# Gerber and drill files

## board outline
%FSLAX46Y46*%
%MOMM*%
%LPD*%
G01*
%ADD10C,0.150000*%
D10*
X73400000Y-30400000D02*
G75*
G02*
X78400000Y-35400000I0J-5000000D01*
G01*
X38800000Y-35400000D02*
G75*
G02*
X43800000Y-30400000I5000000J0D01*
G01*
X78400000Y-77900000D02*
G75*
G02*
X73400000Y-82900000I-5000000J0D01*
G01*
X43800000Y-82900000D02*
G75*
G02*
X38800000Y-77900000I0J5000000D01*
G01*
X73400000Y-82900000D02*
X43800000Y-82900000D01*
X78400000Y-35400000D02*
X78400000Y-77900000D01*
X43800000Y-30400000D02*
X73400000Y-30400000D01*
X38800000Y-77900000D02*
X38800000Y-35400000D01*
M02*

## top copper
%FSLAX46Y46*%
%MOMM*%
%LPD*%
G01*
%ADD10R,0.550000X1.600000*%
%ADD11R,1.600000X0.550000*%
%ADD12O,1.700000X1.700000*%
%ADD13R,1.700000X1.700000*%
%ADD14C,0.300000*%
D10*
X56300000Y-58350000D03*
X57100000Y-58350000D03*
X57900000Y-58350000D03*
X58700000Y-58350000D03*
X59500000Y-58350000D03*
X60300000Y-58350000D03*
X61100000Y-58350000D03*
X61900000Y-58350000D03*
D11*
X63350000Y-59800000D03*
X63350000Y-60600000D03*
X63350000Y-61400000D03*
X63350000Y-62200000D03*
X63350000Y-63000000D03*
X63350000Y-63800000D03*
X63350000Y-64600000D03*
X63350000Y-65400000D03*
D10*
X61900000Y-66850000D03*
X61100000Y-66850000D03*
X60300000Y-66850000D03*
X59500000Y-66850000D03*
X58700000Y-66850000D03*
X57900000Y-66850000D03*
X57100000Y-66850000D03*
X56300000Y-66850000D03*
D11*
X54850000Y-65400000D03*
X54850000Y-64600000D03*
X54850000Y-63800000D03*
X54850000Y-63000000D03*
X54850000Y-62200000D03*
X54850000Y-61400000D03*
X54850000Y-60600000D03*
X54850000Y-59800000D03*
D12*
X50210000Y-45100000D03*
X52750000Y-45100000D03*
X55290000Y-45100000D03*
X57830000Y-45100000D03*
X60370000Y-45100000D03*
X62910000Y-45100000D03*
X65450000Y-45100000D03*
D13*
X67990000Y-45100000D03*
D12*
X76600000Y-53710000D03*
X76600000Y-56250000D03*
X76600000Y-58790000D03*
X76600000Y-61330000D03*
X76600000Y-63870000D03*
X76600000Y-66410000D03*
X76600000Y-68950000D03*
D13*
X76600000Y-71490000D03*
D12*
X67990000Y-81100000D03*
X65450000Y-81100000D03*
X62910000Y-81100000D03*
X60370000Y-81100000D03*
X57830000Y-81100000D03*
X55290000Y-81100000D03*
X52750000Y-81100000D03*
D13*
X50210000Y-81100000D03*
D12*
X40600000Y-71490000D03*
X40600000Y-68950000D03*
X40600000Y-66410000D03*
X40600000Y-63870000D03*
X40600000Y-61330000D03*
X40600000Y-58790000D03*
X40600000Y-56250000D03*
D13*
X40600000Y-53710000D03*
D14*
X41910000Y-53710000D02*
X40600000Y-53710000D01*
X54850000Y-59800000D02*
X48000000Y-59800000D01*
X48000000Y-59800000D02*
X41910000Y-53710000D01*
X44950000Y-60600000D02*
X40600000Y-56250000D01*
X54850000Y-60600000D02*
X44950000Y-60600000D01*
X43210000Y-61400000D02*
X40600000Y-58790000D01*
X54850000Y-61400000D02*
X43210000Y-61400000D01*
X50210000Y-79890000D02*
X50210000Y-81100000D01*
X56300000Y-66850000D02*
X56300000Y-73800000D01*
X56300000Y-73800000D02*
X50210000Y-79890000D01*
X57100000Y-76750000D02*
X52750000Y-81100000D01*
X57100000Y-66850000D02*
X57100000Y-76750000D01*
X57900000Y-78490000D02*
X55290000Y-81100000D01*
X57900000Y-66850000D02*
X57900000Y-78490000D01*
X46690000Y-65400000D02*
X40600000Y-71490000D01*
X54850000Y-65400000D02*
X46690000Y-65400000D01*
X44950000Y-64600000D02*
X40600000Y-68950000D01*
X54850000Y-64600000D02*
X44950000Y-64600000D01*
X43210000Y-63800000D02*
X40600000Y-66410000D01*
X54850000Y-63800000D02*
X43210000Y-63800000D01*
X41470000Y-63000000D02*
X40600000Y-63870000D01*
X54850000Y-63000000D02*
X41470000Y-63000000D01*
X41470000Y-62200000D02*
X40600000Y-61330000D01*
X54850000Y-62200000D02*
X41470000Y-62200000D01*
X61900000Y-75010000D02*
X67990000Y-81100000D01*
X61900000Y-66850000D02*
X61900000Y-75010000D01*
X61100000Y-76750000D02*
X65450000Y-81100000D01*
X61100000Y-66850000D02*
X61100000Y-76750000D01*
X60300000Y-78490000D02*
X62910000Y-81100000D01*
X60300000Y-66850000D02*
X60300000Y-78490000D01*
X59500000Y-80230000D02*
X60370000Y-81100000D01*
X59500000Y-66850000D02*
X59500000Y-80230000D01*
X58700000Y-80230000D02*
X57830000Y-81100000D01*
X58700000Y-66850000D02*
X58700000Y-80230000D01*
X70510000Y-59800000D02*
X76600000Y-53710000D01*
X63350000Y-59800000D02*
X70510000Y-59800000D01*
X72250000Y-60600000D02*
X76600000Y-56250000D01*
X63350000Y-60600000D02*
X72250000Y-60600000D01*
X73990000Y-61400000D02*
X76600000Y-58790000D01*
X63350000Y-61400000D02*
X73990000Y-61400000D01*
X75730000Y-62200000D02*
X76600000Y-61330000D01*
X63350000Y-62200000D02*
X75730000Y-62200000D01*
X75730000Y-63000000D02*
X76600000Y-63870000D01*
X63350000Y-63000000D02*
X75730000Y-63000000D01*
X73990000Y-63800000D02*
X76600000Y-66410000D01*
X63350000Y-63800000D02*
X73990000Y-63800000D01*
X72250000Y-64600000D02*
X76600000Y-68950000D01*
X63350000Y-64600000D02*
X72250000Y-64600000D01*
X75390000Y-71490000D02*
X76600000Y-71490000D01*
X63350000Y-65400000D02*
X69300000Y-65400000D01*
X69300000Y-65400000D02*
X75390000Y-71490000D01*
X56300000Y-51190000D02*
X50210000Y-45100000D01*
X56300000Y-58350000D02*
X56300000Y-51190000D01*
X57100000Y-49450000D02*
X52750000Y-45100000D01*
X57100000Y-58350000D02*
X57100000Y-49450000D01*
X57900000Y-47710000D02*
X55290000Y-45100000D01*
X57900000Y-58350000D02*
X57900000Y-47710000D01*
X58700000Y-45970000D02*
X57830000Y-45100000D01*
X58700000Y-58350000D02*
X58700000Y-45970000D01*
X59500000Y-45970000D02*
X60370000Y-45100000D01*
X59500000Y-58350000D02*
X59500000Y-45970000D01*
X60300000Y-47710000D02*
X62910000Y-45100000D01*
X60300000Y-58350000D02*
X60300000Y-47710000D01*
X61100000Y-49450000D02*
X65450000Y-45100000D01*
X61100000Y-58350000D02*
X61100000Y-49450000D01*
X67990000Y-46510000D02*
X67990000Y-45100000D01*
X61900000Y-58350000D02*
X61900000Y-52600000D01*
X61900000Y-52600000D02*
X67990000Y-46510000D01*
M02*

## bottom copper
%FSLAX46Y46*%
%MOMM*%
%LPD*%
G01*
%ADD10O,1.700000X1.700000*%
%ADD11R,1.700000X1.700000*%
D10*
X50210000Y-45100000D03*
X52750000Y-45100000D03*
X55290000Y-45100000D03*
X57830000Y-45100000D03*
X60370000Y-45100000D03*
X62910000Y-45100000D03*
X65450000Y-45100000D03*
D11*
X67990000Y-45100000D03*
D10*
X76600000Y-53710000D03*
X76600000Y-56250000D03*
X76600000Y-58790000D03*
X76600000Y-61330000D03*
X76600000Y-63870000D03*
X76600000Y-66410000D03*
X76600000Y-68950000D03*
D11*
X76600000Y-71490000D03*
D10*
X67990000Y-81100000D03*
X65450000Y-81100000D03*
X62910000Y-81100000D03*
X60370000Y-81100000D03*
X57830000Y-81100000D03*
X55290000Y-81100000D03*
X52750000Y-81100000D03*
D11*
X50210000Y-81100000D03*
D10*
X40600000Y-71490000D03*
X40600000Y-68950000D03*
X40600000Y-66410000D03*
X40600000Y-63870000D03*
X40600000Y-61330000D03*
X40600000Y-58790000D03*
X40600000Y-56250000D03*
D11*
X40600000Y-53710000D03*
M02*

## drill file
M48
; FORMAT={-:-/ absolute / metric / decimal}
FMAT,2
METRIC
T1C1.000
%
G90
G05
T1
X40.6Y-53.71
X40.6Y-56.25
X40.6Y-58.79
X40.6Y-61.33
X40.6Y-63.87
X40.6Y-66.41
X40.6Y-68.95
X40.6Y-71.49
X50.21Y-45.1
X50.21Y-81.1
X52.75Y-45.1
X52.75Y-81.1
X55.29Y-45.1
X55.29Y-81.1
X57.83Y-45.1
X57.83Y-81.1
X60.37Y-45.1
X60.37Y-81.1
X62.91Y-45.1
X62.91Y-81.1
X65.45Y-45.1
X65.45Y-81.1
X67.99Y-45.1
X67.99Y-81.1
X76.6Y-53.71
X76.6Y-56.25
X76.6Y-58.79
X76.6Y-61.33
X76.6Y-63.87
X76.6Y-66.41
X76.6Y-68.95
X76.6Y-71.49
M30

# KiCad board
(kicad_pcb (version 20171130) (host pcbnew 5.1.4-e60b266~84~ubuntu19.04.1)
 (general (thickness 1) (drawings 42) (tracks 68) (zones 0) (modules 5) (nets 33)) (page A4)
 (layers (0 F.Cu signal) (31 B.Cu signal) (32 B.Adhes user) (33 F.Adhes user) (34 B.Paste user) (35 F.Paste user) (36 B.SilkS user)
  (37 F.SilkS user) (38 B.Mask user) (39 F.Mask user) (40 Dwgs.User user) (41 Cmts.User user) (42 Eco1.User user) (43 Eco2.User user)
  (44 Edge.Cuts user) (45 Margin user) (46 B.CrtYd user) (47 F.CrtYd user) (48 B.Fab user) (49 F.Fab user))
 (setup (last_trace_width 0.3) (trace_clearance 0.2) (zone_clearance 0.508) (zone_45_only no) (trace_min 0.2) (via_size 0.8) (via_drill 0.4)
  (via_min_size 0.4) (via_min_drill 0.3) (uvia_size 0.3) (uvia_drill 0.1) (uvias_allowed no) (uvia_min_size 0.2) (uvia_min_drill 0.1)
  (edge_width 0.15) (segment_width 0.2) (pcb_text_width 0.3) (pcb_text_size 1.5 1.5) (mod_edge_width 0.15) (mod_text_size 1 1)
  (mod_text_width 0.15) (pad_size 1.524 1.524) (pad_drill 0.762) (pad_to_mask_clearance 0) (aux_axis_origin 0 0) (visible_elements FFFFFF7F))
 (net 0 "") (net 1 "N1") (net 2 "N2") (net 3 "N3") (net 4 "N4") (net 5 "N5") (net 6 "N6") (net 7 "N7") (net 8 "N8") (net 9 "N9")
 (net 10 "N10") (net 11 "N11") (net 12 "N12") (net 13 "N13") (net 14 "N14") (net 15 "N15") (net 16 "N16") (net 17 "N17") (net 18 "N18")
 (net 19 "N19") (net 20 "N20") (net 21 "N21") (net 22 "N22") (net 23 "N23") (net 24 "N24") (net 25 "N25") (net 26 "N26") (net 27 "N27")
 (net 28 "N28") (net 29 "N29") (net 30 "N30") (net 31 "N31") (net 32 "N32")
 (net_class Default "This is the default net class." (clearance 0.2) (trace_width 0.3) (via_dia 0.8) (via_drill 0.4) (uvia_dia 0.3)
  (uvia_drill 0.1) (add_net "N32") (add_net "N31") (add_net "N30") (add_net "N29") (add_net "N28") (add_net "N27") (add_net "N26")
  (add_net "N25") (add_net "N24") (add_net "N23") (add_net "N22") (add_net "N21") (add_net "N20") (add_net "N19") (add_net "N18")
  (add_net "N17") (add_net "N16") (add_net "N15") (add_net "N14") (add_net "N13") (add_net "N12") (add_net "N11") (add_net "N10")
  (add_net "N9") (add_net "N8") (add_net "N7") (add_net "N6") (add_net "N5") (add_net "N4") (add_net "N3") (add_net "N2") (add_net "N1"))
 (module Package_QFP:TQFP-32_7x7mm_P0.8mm (layer F.Cu) (at 59.1 62.6)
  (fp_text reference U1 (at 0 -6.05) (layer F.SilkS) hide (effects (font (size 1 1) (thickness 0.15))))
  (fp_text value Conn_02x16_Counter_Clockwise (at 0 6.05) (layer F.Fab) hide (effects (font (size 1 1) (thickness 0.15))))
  (pad 32 smd rect (at -2.8 -4.25 90) (size 1.6 0.55) (layers F.Cu F.Paste F.Mask) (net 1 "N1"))
  (pad 31 smd rect (at -2 -4.25 90) (size 1.6 0.55) (layers F.Cu F.Paste F.Mask) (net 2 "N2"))
  (pad 30 smd rect (at -1.2 -4.25 90) (size 1.6 0.55) (layers F.Cu F.Paste F.Mask) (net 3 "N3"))
  (pad 29 smd rect (at -0.4 -4.25 90) (size 1.6 0.55) (layers F.Cu F.Paste F.Mask) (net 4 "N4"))
  (pad 28 smd rect (at 0.4 -4.25 90) (size 1.6 0.55) (layers F.Cu F.Paste F.Mask) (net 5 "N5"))
  (pad 27 smd rect (at 1.2 -4.25 90) (size 1.6 0.55) (layers F.Cu F.Paste F.Mask) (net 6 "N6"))
  (pad 26 smd rect (at 2 -4.25 90) (size 1.6 0.55) (layers F.Cu F.Paste F.Mask) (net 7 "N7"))
  (pad 25 smd rect (at 2.8 -4.25 90) (size 1.6 0.55) (layers F.Cu F.Paste F.Mask) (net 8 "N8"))
  (pad 24 smd rect (at 4.25 -2.8) (size 1.6 0.55) (layers F.Cu F.Paste F.Mask) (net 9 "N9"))
  (pad 23 smd rect (at 4.25 -2) (size 1.6 0.55) (layers F.Cu F.Paste F.Mask) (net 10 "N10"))
  (pad 22 smd rect (at 4.25 -1.2) (size 1.6 0.55) (layers F.Cu F.Paste F.Mask) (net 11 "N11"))
  (pad 21 smd rect (at 4.25 -0.4) (size 1.6 0.55) (layers F.Cu F.Paste F.Mask) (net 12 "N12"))
  (pad 20 smd rect (at 4.25 0.4) (size 1.6 0.55) (layers F.Cu F.Paste F.Mask) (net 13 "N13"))
  (pad 19 smd rect (at 4.25 1.2) (size 1.6 0.55) (layers F.Cu F.Paste F.Mask) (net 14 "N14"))
  (pad 18 smd rect (at 4.25 2) (size 1.6 0.55) (layers F.Cu F.Paste F.Mask) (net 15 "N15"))
  (pad 17 smd rect (at 4.25 2.8) (size 1.6 0.55) (layers F.Cu F.Paste F.Mask) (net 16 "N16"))
  (pad 16 smd rect (at 2.8 4.25 90) (size 1.6 0.55) (layers F.Cu F.Paste F.Mask) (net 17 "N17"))
  (pad 15 smd rect (at 2 4.25 90) (size 1.6 0.55) (layers F.Cu F.Paste F.Mask) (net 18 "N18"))
  (pad 14 smd rect (at 1.2 4.25 90) (size 1.6 0.55) (layers F.Cu F.Paste F.Mask) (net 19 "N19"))
  (pad 13 smd rect (at 0.4 4.25 90) (size 1.6 0.55) (layers F.Cu F.Paste F.Mask) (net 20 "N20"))
  (pad 12 smd rect (at -0.4 4.25 90) (size 1.6 0.55) (layers F.Cu F.Paste F.Mask) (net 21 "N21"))
  (pad 11 smd rect (at -1.2 4.25 90) (size 1.6 0.55) (layers F.Cu F.Paste F.Mask) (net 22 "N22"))
  (pad 10 smd rect (at -2 4.25 90) (size 1.6 0.55) (layers F.Cu F.Paste F.Mask) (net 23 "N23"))
  (pad 9 smd rect (at -2.8 4.25 90) (size 1.6 0.55) (layers F.Cu F.Paste F.Mask) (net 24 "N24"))
  (pad 8 smd rect (at -4.25 2.8) (size 1.6 0.55) (layers F.Cu F.Paste F.Mask) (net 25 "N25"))
  (pad 7 smd rect (at -4.25 2) (size 1.6 0.55) (layers F.Cu F.Paste F.Mask) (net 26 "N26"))
  (pad 6 smd rect (at -4.25 1.2) (size 1.6 0.55) (layers F.Cu F.Paste F.Mask) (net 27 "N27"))
  (pad 5 smd rect (at -4.25 0.4) (size 1.6 0.55) (layers F.Cu F.Paste F.Mask) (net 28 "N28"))
  (pad 4 smd rect (at -4.25 -0.4) (size 1.6 0.55) (layers F.Cu F.Paste F.Mask) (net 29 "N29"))
  (pad 3 smd rect (at -4.25 -1.2) (size 1.6 0.55) (layers F.Cu F.Paste F.Mask) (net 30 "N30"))
  (pad 2 smd rect (at -4.25 -2) (size 1.6 0.55) (layers F.Cu F.Paste F.Mask) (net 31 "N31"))
  (pad 1 smd rect (at -4.25 -2.8) (size 1.6 0.55) (layers F.Cu F.Paste F.Mask) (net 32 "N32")))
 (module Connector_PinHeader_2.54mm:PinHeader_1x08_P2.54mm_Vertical (layer F.Cu) (at 67.99 45.1 270)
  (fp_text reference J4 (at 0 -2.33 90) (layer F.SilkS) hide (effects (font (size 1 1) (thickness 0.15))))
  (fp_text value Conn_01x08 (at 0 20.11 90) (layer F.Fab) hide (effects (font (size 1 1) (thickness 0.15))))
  (pad 8 thru_hole oval (at 0 17.78 270) (size 1.7 1.7) (drill 1) (layers *.Cu *.Mask) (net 1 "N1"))
  (pad 7 thru_hole oval (at 0 15.24 270) (size 1.7 1.7) (drill 1) (layers *.Cu *.Mask) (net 2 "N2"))
  (pad 6 thru_hole oval (at 0 12.7 270) (size 1.7 1.7) (drill 1) (layers *.Cu *.Mask) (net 3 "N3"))
  (pad 5 thru_hole oval (at 0 10.16 270) (size 1.7 1.7) (drill 1) (layers *.Cu *.Mask) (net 4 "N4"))
  (pad 4 thru_hole oval (at 0 7.62 270) (size 1.7 1.7) (drill 1) (layers *.Cu *.Mask) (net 5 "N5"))
  (pad 3 thru_hole oval (at 0 5.08 270) (size 1.7 1.7) (drill 1) (layers *.Cu *.Mask) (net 6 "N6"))
  (pad 2 thru_hole oval (at 0 2.54 270) (size 1.7 1.7) (drill 1) (layers *.Cu *.Mask) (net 7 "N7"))
  (pad 1 thru_hole rect (at 0 0 270) (size 1.7 1.7) (drill 1) (layers *.Cu *.Mask) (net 8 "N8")))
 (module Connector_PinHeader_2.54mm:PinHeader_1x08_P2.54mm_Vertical (layer F.Cu) (at 76.6 71.49 180)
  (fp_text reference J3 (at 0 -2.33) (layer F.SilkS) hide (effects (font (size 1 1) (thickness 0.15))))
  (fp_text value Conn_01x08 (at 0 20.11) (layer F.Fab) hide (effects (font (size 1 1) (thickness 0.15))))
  (pad 8 thru_hole oval (at 0 17.78 180) (size 1.7 1.7) (drill 1) (layers *.Cu *.Mask) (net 9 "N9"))
  (pad 7 thru_hole oval (at 0 15.24 180) (size 1.7 1.7) (drill 1) (layers *.Cu *.Mask) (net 10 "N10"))
  (pad 6 thru_hole oval (at 0 12.7 180) (size 1.7 1.7) (drill 1) (layers *.Cu *.Mask) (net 11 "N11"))
  (pad 5 thru_hole oval (at 0 10.16 180) (size 1.7 1.7) (drill 1) (layers *.Cu *.Mask) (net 12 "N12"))
  (pad 4 thru_hole oval (at 0 7.62 180) (size 1.7 1.7) (drill 1) (layers *.Cu *.Mask) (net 13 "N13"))
  (pad 3 thru_hole oval (at 0 5.08 180) (size 1.7 1.7) (drill 1) (layers *.Cu *.Mask) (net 14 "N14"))
  (pad 2 thru_hole oval (at 0 2.54 180) (size 1.7 1.7) (drill 1) (layers *.Cu *.Mask) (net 15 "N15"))
  (pad 1 thru_hole rect (at 0 0 180) (size 1.7 1.7) (drill 1) (layers *.Cu *.Mask) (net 16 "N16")))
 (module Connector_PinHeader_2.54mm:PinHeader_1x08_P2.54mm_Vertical (layer F.Cu) (at 50.21 81.1 90)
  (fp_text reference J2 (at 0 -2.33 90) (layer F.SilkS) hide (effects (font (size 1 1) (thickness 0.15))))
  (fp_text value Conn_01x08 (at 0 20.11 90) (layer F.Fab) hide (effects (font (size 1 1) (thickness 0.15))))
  (pad 8 thru_hole oval (at 0 17.78 90) (size 1.7 1.7) (drill 1) (layers *.Cu *.Mask) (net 17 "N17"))
  (pad 7 thru_hole oval (at 0 15.24 90) (size 1.7 1.7) (drill 1) (layers *.Cu *.Mask) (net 18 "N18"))
  (pad 6 thru_hole oval (at 0 12.7 90) (size 1.7 1.7) (drill 1) (layers *.Cu *.Mask) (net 19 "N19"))
  (pad 5 thru_hole oval (at 0 10.16 90) (size 1.7 1.7) (drill 1) (layers *.Cu *.Mask) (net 20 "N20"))
  (pad 4 thru_hole oval (at 0 7.62 90) (size 1.7 1.7) (drill 1) (layers *.Cu *.Mask) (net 21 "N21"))
  (pad 3 thru_hole oval (at 0 5.08 90) (size 1.7 1.7) (drill 1) (layers *.Cu *.Mask) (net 22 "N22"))
  (pad 2 thru_hole oval (at 0 2.54 90) (size 1.7 1.7) (drill 1) (layers *.Cu *.Mask) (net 23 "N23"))
  (pad 1 thru_hole rect (at 0 0 90) (size 1.7 1.7) (drill 1) (layers *.Cu *.Mask) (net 24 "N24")))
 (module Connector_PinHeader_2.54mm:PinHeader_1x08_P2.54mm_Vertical (layer F.Cu) (at 40.6 53.71)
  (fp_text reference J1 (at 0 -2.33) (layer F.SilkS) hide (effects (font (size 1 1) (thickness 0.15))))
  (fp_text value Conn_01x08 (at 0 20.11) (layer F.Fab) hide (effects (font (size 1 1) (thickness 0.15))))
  (pad 8 thru_hole oval (at 0 17.78) (size 1.7 1.7) (drill 1) (layers *.Cu *.Mask) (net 25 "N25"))
  (pad 7 thru_hole oval (at 0 15.24) (size 1.7 1.7) (drill 1) (layers *.Cu *.Mask) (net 26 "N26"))
  (pad 6 thru_hole oval (at 0 12.7) (size 1.7 1.7) (drill 1) (layers *.Cu *.Mask) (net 27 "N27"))
  (pad 5 thru_hole oval (at 0 10.16) (size 1.7 1.7) (drill 1) (layers *.Cu *.Mask) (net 28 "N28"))
  (pad 4 thru_hole oval (at 0 7.62) (size 1.7 1.7) (drill 1) (layers *.Cu *.Mask) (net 29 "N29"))
  (pad 3 thru_hole oval (at 0 5.08) (size 1.7 1.7) (drill 1) (layers *.Cu *.Mask) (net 30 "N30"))
  (pad 2 thru_hole oval (at 0 2.54) (size 1.7 1.7) (drill 1) (layers *.Cu *.Mask) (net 31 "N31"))
  (pad 1 thru_hole rect (at 0 0) (size 1.7 1.7) (drill 1) (layers *.Cu *.Mask) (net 32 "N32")))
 (gr_arc (start 73.4 35.4) (end 78.4 35.4) (angle -90) (layer Edge.Cuts) (width 0.15))
 (gr_arc (start 43.8 35.4) (end 43.8 30.4) (angle -90) (layer Edge.Cuts) (width 0.15))
 (gr_arc (start 73.4 77.9) (end 73.4 82.9) (angle -90) (layer Edge.Cuts) (width 0.15))
 (gr_arc (start 43.8 77.9) (end 38.8 77.9) (angle -90) (layer Edge.Cuts) (width 0.15))
 (gr_line (start 73.4 82.9) (end 43.8 82.9) (layer Edge.Cuts) (width 0.15))
 (gr_line (start 78.4 35.4) (end 78.4 77.9) (layer Edge.Cuts) (width 0.15))
 (gr_line (start 43.8 30.4) (end 73.4 30.4) (layer Edge.Cuts) (width 0.15))
 (gr_line (start 38.8 77.9) (end 38.8 35.4) (layer Edge.Cuts) (width 0.15))
 (segment (start 41.91 53.71) (end 40.6 53.71) (width 0.3) (layer F.Cu) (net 32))
 (segment (start 54.85 59.8) (end 48 59.8) (width 0.3) (layer F.Cu) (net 32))
 (segment (start 48 59.8) (end 41.91 53.71) (width 0.3) (layer F.Cu) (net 32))
 (segment (start 44.95 60.6) (end 40.6 56.25) (width 0.3) (layer F.Cu) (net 31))
 (segment (start 54.85 60.6) (end 44.95 60.6) (width 0.3) (layer F.Cu) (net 31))
 (segment (start 43.21 61.4) (end 40.6 58.79) (width 0.3) (layer F.Cu) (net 30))
 (segment (start 54.85 61.4) (end 43.21 61.4) (width 0.3) (layer F.Cu) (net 30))
 (segment (start 50.21 79.89) (end 50.21 81.1) (width 0.3) (layer F.Cu) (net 24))
 (segment (start 56.3 66.85) (end 56.3 73.8) (width 0.3) (layer F.Cu) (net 24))
 (segment (start 56.3 73.8) (end 50.21 79.89) (width 0.3) (layer F.Cu) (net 24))
 (segment (start 57.1 76.75) (end 52.75 81.1) (width 0.3) (layer F.Cu) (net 23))
 (segment (start 57.1 66.85) (end 57.1 76.75) (width 0.3) (layer F.Cu) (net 23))
 (segment (start 57.9 78.49) (end 55.29 81.1) (width 0.3) (layer F.Cu) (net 22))
 (segment (start 57.9 66.85) (end 57.9 78.49) (width 0.3) (layer F.Cu) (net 22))
 (segment (start 46.69 65.4) (end 40.6 71.49) (width 0.3) (layer F.Cu) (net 25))
 (segment (start 54.85 65.4) (end 46.69 65.4) (width 0.3) (layer F.Cu) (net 25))
 (segment (start 44.95 64.6) (end 40.6 68.95) (width 0.3) (layer F.Cu) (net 26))
 (segment (start 54.85 64.6) (end 44.95 64.6) (width 0.3) (layer F.Cu) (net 26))
 (segment (start 43.21 63.8) (end 40.6 66.41) (width 0.3) (layer F.Cu) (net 27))
 (segment (start 54.85 63.8) (end 43.21 63.8) (width 0.3) (layer F.Cu) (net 27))
 (segment (start 41.47 63) (end 40.6 63.87) (width 0.3) (layer F.Cu) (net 28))
 (segment (start 54.85 63) (end 41.47 63) (width 0.3) (layer F.Cu) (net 28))
 (segment (start 41.47 62.2) (end 40.6 61.33) (width 0.3) (layer F.Cu) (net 29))
 (segment (start 54.85 62.2) (end 41.47 62.2) (width 0.3) (layer F.Cu) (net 29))
 (segment (start 61.9 75.01) (end 67.99 81.1) (width 0.3) (layer F.Cu) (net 17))
 (segment (start 61.9 66.85) (end 61.9 75.01) (width 0.3) (layer F.Cu) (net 17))
 (segment (start 61.1 76.75) (end 65.45 81.1) (width 0.3) (layer F.Cu) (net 18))
 (segment (start 61.1 66.85) (end 61.1 76.75) (width 0.3) (layer F.Cu) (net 18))
 (segment (start 60.3 78.49) (end 62.91 81.1) (width 0.3) (layer F.Cu) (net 19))
 (segment (start 60.3 66.85) (end 60.3 78.49) (width 0.3) (layer F.Cu) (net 19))
 (segment (start 59.5 80.23) (end 60.37 81.1) (width 0.3) (layer F.Cu) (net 20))
 (segment (start 59.5 66.85) (end 59.5 80.23) (width 0.3) (layer F.Cu) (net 20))
 (segment (start 58.7 80.23) (end 57.83 81.1) (width 0.3) (layer F.Cu) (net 21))
 (segment (start 58.7 66.85) (end 58.7 80.23) (width 0.3) (layer F.Cu) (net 21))
 (segment (start 70.51 59.8) (end 76.6 53.71) (width 0.3) (layer F.Cu) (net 9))
 (segment (start 63.35 59.8) (end 70.51 59.8) (width 0.3) (layer F.Cu) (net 9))
 (segment (start 72.25 60.6) (end 76.6 56.25) (width 0.3) (layer F.Cu) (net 10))
 (segment (start 63.35 60.6) (end 72.25 60.6) (width 0.3) (layer F.Cu) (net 10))
 (segment (start 73.99 61.4) (end 76.6 58.79) (width 0.3) (layer F.Cu) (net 11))
 (segment (start 63.35 61.4) (end 73.99 61.4) (width 0.3) (layer F.Cu) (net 11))
 (segment (start 75.73 62.2) (end 76.6 61.33) (width 0.3) (layer F.Cu) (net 12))
 (segment (start 63.35 62.2) (end 75.73 62.2) (width 0.3) (layer F.Cu) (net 12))
 (segment (start 75.73 63) (end 76.6 63.87) (width 0.3) (layer F.Cu) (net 13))
 (segment (start 63.35 63) (end 75.73 63) (width 0.3) (layer F.Cu) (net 13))
 (segment (start 73.99 63.8) (end 76.6 66.41) (width 0.3) (layer F.Cu) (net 14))
 (segment (start 63.35 63.8) (end 73.99 63.8) (width 0.3) (layer F.Cu) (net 14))
 (segment (start 72.25 64.6) (end 76.6 68.95) (width 0.3) (layer F.Cu) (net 15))
 (segment (start 63.35 64.6) (end 72.25 64.6) (width 0.3) (layer F.Cu) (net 15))
 (segment (start 75.39 71.49) (end 76.6 71.49) (width 0.3) (layer F.Cu) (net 16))
 (segment (start 63.35 65.4) (end 69.3 65.4) (width 0.3) (layer F.Cu) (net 16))
 (segment (start 69.3 65.4) (end 75.39 71.49) (width 0.3) (layer F.Cu) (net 16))
 (segment (start 56.3 51.19) (end 50.21 45.1) (width 0.3) (layer F.Cu) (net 1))
 (segment (start 56.3 58.35) (end 56.3 51.19) (width 0.3) (layer F.Cu) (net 1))
 (segment (start 57.1 49.45) (end 52.75 45.1) (width 0.3) (layer F.Cu) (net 2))
 (segment (start 57.1 58.35) (end 57.1 49.45) (width 0.3) (layer F.Cu) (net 2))
 (segment (start 57.9 47.71) (end 55.29 45.1) (width 0.3) (layer F.Cu) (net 3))
 (segment (start 57.9 58.35) (end 57.9 47.71) (width 0.3) (layer F.Cu) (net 3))
 (segment (start 58.7 45.97) (end 57.83 45.1) (width 0.3) (layer F.Cu) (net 4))
 (segment (start 58.7 58.35) (end 58.7 45.97) (width 0.3) (layer F.Cu) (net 4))
 (segment (start 59.5 45.97) (end 60.37 45.1) (width 0.3) (layer F.Cu) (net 5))
 (segment (start 59.5 58.35) (end 59.5 45.97) (width 0.3) (layer F.Cu) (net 5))
 (segment (start 60.3 47.71) (end 62.91 45.1) (width 0.3) (layer F.Cu) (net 6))
 (segment (start 60.3 58.35) (end 60.3 47.71) (width 0.3) (layer F.Cu) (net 6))
 (segment (start 61.1 49.45) (end 65.45 45.1) (width 0.3) (layer F.Cu) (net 7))
 (segment (start 61.1 58.35) (end 61.1 49.45) (width 0.3) (layer F.Cu) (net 7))
 (segment (start 67.99 46.51) (end 67.99 45.1) (width 0.3) (layer F.Cu) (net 8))
 (segment (start 61.9 58.35) (end 61.9 52.6) (width 0.3) (layer F.Cu) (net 8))
 (segment (start 61.9 52.6) (end 67.99 46.51) (width 0.3) (layer F.Cu) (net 8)))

